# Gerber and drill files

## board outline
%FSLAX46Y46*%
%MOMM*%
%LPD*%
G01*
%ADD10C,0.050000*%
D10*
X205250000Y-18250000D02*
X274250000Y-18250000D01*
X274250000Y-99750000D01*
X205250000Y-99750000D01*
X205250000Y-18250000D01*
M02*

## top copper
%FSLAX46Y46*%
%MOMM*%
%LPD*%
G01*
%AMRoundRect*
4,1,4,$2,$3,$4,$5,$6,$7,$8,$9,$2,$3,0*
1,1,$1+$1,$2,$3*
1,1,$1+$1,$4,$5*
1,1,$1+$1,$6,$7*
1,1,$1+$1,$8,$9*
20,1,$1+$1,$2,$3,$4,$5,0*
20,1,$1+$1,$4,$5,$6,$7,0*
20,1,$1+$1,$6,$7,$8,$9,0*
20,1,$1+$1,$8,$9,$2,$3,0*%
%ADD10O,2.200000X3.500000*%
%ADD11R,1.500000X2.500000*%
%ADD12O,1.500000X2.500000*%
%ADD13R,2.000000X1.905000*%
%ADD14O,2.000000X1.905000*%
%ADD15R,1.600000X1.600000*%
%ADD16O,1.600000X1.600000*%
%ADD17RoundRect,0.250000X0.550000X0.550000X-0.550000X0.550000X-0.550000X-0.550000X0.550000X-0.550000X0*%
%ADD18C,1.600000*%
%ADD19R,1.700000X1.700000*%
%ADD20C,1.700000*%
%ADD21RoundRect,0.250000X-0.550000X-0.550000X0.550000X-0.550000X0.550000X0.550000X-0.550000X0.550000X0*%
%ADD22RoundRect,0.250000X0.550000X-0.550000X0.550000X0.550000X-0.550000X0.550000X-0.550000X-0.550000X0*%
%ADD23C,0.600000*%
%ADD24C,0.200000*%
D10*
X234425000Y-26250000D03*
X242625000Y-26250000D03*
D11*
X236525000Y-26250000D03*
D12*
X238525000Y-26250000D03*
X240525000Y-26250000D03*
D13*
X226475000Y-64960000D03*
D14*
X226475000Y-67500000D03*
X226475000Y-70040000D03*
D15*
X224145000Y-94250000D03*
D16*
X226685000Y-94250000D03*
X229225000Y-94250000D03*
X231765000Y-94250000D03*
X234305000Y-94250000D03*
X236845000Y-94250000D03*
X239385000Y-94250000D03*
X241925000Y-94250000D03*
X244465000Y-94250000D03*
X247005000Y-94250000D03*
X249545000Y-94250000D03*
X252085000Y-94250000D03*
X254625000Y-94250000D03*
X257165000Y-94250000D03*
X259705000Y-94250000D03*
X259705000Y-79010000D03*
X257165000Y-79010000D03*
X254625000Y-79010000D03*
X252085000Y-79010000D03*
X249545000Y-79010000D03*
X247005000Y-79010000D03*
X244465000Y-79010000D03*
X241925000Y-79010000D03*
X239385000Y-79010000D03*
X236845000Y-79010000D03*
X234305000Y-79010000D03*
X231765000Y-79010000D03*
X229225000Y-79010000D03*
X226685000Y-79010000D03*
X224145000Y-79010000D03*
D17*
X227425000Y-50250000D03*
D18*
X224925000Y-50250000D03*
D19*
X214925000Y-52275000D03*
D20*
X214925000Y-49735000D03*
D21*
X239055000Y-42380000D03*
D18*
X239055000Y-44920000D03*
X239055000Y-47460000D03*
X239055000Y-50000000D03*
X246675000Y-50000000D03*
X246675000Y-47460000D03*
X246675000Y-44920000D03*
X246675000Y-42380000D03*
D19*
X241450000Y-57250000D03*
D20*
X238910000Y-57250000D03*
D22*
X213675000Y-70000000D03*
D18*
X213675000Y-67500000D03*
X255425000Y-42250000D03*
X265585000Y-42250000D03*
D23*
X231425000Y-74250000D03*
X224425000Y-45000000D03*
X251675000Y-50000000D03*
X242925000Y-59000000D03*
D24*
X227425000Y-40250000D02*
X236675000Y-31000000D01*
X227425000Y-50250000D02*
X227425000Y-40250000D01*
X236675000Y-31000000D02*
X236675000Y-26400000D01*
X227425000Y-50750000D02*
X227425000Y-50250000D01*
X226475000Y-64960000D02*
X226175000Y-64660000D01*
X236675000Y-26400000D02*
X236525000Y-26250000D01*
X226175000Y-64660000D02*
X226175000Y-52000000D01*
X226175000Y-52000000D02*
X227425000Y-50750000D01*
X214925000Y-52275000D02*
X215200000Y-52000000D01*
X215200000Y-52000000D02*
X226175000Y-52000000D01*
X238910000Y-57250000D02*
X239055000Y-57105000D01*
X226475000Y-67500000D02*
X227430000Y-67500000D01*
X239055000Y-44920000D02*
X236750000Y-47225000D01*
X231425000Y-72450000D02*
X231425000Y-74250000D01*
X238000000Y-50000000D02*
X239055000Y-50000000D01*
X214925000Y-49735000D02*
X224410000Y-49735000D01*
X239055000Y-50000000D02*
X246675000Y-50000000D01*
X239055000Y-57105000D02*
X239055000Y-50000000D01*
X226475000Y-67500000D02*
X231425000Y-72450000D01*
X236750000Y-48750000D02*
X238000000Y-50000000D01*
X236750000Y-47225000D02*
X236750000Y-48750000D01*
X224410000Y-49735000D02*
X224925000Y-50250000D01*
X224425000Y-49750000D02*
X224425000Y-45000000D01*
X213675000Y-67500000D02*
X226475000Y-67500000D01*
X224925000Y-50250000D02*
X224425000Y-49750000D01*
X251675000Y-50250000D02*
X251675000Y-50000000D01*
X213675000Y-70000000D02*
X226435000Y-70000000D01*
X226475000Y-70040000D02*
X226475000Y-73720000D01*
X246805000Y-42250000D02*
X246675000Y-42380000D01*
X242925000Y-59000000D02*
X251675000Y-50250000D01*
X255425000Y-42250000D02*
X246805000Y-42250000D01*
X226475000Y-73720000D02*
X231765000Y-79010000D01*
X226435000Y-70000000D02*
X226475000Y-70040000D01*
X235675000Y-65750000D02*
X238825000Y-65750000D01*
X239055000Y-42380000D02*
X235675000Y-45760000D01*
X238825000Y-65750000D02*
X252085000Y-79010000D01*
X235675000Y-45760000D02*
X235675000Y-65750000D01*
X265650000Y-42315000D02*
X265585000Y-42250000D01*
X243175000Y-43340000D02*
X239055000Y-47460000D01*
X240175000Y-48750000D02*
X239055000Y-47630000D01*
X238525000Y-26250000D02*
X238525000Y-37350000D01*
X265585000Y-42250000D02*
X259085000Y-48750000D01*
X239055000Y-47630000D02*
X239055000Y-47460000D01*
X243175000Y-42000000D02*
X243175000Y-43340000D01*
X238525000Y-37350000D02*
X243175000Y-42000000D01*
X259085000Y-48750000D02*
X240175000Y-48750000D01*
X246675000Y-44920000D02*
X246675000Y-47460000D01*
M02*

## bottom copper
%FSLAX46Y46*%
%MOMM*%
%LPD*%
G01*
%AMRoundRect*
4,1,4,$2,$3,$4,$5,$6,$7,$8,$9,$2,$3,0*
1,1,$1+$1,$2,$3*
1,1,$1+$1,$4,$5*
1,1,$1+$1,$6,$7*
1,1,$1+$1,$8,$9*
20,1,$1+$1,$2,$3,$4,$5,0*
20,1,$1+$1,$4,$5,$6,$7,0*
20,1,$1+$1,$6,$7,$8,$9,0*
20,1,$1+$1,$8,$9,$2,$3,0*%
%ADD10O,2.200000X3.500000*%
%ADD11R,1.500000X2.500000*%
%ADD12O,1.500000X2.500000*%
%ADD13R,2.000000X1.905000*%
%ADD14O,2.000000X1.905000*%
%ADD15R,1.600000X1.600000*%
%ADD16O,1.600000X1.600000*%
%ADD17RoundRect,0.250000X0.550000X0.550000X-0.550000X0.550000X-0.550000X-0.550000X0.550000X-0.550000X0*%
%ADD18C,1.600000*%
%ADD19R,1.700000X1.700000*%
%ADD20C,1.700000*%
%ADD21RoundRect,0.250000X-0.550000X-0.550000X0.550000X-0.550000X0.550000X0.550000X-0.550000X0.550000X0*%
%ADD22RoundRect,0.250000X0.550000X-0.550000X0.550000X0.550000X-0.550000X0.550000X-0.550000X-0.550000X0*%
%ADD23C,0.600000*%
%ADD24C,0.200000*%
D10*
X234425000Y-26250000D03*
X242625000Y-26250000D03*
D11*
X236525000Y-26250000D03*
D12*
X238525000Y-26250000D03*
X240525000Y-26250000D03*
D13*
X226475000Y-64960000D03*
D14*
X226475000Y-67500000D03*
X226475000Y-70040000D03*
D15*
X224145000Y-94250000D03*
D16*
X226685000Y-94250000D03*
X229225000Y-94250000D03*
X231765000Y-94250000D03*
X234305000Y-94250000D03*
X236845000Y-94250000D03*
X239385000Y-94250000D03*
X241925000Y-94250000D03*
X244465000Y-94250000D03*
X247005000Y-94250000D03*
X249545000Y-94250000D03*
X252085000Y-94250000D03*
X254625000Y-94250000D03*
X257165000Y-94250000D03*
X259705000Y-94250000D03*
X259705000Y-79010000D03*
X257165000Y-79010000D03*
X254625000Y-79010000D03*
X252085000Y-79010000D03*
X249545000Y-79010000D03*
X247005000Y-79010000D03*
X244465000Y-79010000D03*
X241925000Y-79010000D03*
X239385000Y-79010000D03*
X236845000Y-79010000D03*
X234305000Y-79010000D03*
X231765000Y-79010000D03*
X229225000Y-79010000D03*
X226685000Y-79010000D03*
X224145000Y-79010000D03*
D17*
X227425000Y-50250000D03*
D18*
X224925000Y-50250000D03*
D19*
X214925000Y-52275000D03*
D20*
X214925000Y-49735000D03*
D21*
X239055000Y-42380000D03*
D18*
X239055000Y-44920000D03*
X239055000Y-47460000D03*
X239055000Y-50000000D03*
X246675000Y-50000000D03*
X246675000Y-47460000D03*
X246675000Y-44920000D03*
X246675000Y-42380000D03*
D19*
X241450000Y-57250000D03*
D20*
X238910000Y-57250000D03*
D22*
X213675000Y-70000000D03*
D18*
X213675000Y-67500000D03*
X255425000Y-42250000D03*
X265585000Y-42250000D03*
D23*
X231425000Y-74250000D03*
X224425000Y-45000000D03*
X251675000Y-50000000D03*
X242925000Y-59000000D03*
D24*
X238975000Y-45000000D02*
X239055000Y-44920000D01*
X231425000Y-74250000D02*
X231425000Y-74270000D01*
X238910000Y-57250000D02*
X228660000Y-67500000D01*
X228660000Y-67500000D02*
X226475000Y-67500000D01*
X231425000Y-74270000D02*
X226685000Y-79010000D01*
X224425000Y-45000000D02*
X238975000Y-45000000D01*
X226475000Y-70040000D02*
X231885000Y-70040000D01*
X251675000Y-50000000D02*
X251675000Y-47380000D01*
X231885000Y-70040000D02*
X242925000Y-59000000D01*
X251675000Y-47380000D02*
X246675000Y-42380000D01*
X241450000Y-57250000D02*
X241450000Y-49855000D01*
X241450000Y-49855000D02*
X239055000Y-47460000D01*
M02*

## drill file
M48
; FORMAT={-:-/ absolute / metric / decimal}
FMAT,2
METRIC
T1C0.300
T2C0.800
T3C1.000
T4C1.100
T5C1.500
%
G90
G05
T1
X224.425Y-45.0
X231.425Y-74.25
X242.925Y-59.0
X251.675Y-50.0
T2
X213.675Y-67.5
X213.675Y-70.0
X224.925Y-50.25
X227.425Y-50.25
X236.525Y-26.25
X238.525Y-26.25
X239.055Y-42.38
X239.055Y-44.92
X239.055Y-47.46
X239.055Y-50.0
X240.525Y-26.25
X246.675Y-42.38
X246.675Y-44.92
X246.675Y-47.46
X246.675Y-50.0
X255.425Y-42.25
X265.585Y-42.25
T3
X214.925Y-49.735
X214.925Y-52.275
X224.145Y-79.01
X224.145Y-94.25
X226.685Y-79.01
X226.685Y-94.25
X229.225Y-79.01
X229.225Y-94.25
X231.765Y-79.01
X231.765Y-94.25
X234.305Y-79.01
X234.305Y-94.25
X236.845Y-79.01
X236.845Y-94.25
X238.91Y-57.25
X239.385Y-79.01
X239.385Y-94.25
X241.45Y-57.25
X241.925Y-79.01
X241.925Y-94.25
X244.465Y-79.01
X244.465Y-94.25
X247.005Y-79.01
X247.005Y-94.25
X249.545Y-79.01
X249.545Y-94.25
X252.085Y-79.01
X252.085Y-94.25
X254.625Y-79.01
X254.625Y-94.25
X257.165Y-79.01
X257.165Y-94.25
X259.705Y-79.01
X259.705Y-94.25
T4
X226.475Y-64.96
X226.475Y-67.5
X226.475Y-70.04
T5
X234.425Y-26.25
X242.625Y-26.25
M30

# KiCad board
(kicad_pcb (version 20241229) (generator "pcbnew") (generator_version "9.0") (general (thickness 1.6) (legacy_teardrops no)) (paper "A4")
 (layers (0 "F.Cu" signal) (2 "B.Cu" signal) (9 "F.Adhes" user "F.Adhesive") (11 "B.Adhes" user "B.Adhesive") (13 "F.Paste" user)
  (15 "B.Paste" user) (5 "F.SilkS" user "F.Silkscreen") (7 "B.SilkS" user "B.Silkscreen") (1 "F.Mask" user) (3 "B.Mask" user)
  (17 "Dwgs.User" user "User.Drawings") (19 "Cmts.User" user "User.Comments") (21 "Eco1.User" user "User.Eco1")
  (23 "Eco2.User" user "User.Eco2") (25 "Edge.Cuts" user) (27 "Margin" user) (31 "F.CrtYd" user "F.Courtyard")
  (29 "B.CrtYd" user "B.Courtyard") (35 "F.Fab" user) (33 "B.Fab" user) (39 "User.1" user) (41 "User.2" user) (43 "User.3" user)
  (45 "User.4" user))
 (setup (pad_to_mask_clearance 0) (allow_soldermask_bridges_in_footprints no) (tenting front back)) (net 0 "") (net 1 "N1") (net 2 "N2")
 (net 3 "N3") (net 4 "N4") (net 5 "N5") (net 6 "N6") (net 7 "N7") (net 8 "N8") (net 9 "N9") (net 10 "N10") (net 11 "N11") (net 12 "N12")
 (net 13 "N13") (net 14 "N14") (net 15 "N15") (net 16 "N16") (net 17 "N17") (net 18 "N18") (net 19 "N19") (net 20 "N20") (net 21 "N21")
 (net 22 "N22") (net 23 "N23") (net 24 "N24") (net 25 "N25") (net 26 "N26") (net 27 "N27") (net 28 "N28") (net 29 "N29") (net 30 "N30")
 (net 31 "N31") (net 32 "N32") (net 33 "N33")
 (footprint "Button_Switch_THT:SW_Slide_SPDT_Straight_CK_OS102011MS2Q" (layer "F.Cu") (at 236.525 26.25)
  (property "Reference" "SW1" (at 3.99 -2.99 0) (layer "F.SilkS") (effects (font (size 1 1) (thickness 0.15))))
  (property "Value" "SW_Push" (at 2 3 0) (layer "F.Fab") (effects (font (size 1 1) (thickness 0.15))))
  (pad "" thru_hole oval (at -2.1 0) (size 2.2 3.5) (drill 1.5) (layers "*.Cu" "*.Mask") (remove_unused_layers no))
  (pad "" thru_hole oval (at 6.1 0) (size 2.2 3.5) (drill 1.5) (layers "*.Cu" "*.Mask") (remove_unused_layers no))
  (pad "1" thru_hole rect (at 0 0) (size 1.5 2.5) (drill 0.8) (layers "*.Cu" "*.Mask") (remove_unused_layers no) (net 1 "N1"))
  (pad "2" thru_hole oval (at 2 0) (size 1.5 2.5) (drill 0.8) (layers "*.Cu" "*.Mask") (remove_unused_layers no) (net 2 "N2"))
  (pad "3" thru_hole oval (at 4 0) (size 1.5 2.5) (drill 0.8) (layers "*.Cu" "*.Mask") (remove_unused_layers no)))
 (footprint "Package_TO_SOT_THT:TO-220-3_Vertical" (layer "F.Cu") (at 226.475 64.96 -90)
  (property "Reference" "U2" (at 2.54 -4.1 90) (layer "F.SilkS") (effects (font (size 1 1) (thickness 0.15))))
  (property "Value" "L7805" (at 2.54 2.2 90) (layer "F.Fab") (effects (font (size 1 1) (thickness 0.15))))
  (pad "1" thru_hole rect (at 0 0 270) (size 1.905 2) (drill 1.1) (layers "*.Cu" "*.Mask") (remove_unused_layers no) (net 1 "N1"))
  (pad "2" thru_hole oval (at 2.54 0 270) (size 1.905 2) (drill 1.1) (layers "*.Cu" "*.Mask") (remove_unused_layers no) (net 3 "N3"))
  (pad "3" thru_hole oval (at 5.08 0 270) (size 1.905 2) (drill 1.1) (layers "*.Cu" "*.Mask") (remove_unused_layers no) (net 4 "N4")))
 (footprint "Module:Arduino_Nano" (layer "F.Cu") (at 224.145 94.25 90)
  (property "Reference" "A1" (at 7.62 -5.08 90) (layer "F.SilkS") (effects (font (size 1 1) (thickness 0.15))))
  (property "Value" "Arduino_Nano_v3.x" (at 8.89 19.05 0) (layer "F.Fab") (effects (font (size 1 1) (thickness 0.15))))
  (pad "1" thru_hole rect (at 0 0 90) (size 1.6 1.6) (drill 1) (layers "*.Cu" "*.Mask") (remove_unused_layers no) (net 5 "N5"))
  (pad "2" thru_hole oval (at 0 2.54 90) (size 1.6 1.6) (drill 1) (layers "*.Cu" "*.Mask") (remove_unused_layers no) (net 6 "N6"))
  (pad "3" thru_hole oval (at 0 5.08 90) (size 1.6 1.6) (drill 1) (layers "*.Cu" "*.Mask") (remove_unused_layers no) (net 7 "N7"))
  (pad "4" thru_hole oval (at 0 7.62 90) (size 1.6 1.6) (drill 1) (layers "*.Cu" "*.Mask") (remove_unused_layers no) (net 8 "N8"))
  (pad "5" thru_hole oval (at 0 10.16 90) (size 1.6 1.6) (drill 1) (layers "*.Cu" "*.Mask") (remove_unused_layers no) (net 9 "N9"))
  (pad "6" thru_hole oval (at 0 12.7 90) (size 1.6 1.6) (drill 1) (layers "*.Cu" "*.Mask") (remove_unused_layers no) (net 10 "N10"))
  (pad "7" thru_hole oval (at 0 15.24 90) (size 1.6 1.6) (drill 1) (layers "*.Cu" "*.Mask") (remove_unused_layers no) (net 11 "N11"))
  (pad "8" thru_hole oval (at 0 17.78 90) (size 1.6 1.6) (drill 1) (layers "*.Cu" "*.Mask") (remove_unused_layers no) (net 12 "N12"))
  (pad "9" thru_hole oval (at 0 20.32 90) (size 1.6 1.6) (drill 1) (layers "*.Cu" "*.Mask") (remove_unused_layers no) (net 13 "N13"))
  (pad "10" thru_hole oval (at 0 22.86 90) (size 1.6 1.6) (drill 1) (layers "*.Cu" "*.Mask") (remove_unused_layers no) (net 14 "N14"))
  (pad "11" thru_hole oval (at 0 25.4 90) (size 1.6 1.6) (drill 1) (layers "*.Cu" "*.Mask") (remove_unused_layers no) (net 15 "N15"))
  (pad "12" thru_hole oval (at 0 27.94 90) (size 1.6 1.6) (drill 1) (layers "*.Cu" "*.Mask") (remove_unused_layers no) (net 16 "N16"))
  (pad "13" thru_hole oval (at 0 30.48 90) (size 1.6 1.6) (drill 1) (layers "*.Cu" "*.Mask") (remove_unused_layers no) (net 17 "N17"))
  (pad "14" thru_hole oval (at 0 33.02 90) (size 1.6 1.6) (drill 1) (layers "*.Cu" "*.Mask") (remove_unused_layers no) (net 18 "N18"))
  (pad "15" thru_hole oval (at 0 35.56 90) (size 1.6 1.6) (drill 1) (layers "*.Cu" "*.Mask") (remove_unused_layers no) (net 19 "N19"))
  (pad "16" thru_hole oval (at 15.24 35.56 90) (size 1.6 1.6) (drill 1) (layers "*.Cu" "*.Mask") (remove_unused_layers no) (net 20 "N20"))
  (pad "17" thru_hole oval (at 15.24 33.02 90) (size 1.6 1.6) (drill 1) (layers "*.Cu" "*.Mask") (remove_unused_layers no) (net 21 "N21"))
  (pad "18" thru_hole oval (at 15.24 30.48 90) (size 1.6 1.6) (drill 1) (layers "*.Cu" "*.Mask") (remove_unused_layers no) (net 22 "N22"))
  (pad "19" thru_hole oval (at 15.24 27.94 90) (size 1.6 1.6) (drill 1) (layers "*.Cu" "*.Mask") (remove_unused_layers no) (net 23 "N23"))
  (pad "20" thru_hole oval (at 15.24 25.4 90) (size 1.6 1.6) (drill 1) (layers "*.Cu" "*.Mask") (remove_unused_layers no) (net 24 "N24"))
  (pad "21" thru_hole oval (at 15.24 22.86 90) (size 1.6 1.6) (drill 1) (layers "*.Cu" "*.Mask") (remove_unused_layers no) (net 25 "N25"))
  (pad "22" thru_hole oval (at 15.24 20.32 90) (size 1.6 1.6) (drill 1) (layers "*.Cu" "*.Mask") (remove_unused_layers no) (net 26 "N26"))
  (pad "23" thru_hole oval (at 15.24 17.78 90) (size 1.6 1.6) (drill 1) (layers "*.Cu" "*.Mask") (remove_unused_layers no) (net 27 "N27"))
  (pad "24" thru_hole oval (at 15.24 15.24 90) (size 1.6 1.6) (drill 1) (layers "*.Cu" "*.Mask") (remove_unused_layers no) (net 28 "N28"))
  (pad "25" thru_hole oval (at 15.24 12.7 90) (size 1.6 1.6) (drill 1) (layers "*.Cu" "*.Mask") (remove_unused_layers no) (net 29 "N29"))
  (pad "26" thru_hole oval (at 15.24 10.16 90) (size 1.6 1.6) (drill 1) (layers "*.Cu" "*.Mask") (remove_unused_layers no) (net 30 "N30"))
  (pad "27" thru_hole oval (at 15.24 7.62 90) (size 1.6 1.6) (drill 1) (layers "*.Cu" "*.Mask") (remove_unused_layers no) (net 4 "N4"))
  (pad "28" thru_hole oval (at 15.24 5.08 90) (size 1.6 1.6) (drill 1) (layers "*.Cu" "*.Mask") (remove_unused_layers no) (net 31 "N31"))
  (pad "29" thru_hole oval (at 15.24 2.54 90) (size 1.6 1.6) (drill 1) (layers "*.Cu" "*.Mask") (remove_unused_layers no) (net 3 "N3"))
  (pad "30" thru_hole oval (at 15.24 0 90) (size 1.6 1.6) (drill 1) (layers "*.Cu" "*.Mask") (remove_unused_layers no) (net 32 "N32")))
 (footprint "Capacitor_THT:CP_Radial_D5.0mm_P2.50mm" (layer "F.Cu") (at 227.425 50.25 180)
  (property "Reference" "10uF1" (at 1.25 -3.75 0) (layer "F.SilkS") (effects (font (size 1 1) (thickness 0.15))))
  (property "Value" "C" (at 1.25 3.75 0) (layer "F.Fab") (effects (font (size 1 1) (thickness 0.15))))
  (pad "1" thru_hole roundrect (at 0 0 180) (size 1.6 1.6) (drill 0.8) (layers "*.Cu" "*.Mask") (remove_unused_layers no)
   (roundrect_rratio 0.15625) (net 1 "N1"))
  (pad "2" thru_hole circle (at 2.5 0 180) (size 1.6 1.6) (drill 0.8) (layers "*.Cu" "*.Mask") (remove_unused_layers no) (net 3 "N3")))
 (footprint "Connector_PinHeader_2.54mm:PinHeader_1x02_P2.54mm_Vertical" (layer "F.Cu") (at 214.925 52.275 180)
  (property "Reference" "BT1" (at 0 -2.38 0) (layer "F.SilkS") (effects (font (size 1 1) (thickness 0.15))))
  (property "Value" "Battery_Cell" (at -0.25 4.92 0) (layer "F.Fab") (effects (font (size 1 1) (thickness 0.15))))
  (pad "1" thru_hole rect (at 0 0 180) (size 1.7 1.7) (drill 1) (layers "*.Cu" "*.Mask") (remove_unused_layers no) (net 1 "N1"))
  (pad "2" thru_hole circle (at 0 2.54 180) (size 1.7 1.7) (drill 1) (layers "*.Cu" "*.Mask") (remove_unused_layers no) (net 3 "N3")))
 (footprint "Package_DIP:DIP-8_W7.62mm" (layer "F.Cu") (at 239.055 42.38)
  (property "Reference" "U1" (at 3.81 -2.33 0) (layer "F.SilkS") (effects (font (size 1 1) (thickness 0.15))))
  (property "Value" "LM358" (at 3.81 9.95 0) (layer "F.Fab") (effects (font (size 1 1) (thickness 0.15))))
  (pad "1" thru_hole roundrect (at 0 0) (size 1.6 1.6) (drill 0.8) (layers "*.Cu" "*.Mask") (remove_unused_layers no)
   (roundrect_rratio 0.15625) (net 23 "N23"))
  (pad "2" thru_hole circle (at 0 2.54) (size 1.6 1.6) (drill 0.8) (layers "*.Cu" "*.Mask") (remove_unused_layers no) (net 3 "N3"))
  (pad "3" thru_hole circle (at 0 5.08) (size 1.6 1.6) (drill 0.8) (layers "*.Cu" "*.Mask") (remove_unused_layers no) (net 2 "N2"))
  (pad "4" thru_hole circle (at 0 7.62) (size 1.6 1.6) (drill 0.8) (layers "*.Cu" "*.Mask") (remove_unused_layers no) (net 3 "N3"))
  (pad "5" thru_hole circle (at 7.62 7.62) (size 1.6 1.6) (drill 0.8) (layers "*.Cu" "*.Mask") (remove_unused_layers no) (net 3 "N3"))
  (pad "6" thru_hole circle (at 7.62 5.08) (size 1.6 1.6) (drill 0.8) (layers "*.Cu" "*.Mask") (remove_unused_layers no) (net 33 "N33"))
  (pad "7" thru_hole circle (at 7.62 2.54) (size 1.6 1.6) (drill 0.8) (layers "*.Cu" "*.Mask") (remove_unused_layers no) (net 33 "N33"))
  (pad "8" thru_hole circle (at 7.62 0) (size 1.6 1.6) (drill 0.8) (layers "*.Cu" "*.Mask") (remove_unused_layers no) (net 4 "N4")))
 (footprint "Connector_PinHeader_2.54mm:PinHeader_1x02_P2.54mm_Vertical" (layer "F.Cu") (at 241.45 57.25 -90)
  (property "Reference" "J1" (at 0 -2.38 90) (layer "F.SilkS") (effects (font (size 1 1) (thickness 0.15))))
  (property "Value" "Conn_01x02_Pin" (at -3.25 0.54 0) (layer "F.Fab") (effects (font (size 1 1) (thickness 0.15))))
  (pad "1" thru_hole rect (at 0 0 270) (size 1.7 1.7) (drill 1) (layers "*.Cu" "*.Mask") (remove_unused_layers no) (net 2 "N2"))
  (pad "2" thru_hole circle (at 0 2.54 270) (size 1.7 1.7) (drill 1) (layers "*.Cu" "*.Mask") (remove_unused_layers no) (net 3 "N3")))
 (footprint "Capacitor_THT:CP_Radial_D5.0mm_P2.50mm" (layer "F.Cu") (at 213.675 70 90)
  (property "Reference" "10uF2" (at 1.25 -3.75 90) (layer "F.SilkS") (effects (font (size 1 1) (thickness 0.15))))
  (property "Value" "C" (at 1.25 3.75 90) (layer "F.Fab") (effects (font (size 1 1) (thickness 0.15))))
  (pad "1" thru_hole roundrect (at 0 0 90) (size 1.6 1.6) (drill 0.8) (layers "*.Cu" "*.Mask") (remove_unused_layers no)
   (roundrect_rratio 0.15625) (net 4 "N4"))
  (pad "2" thru_hole circle (at 2.5 0 90) (size 1.6 1.6) (drill 0.8) (layers "*.Cu" "*.Mask") (remove_unused_layers no) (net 3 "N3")))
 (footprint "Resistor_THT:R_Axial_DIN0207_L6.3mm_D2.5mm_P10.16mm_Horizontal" (layer "F.Cu") (at 255.425 42.25)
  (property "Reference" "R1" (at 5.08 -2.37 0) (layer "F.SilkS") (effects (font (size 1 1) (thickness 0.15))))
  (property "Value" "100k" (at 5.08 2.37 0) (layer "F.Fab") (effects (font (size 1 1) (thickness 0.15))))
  (pad "1" thru_hole circle (at 0 0) (size 1.6 1.6) (drill 0.8) (layers "*.Cu" "*.Mask") (remove_unused_layers no) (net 4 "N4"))
  (pad "2" thru_hole circle (at 10.16 0) (size 1.6 1.6) (drill 0.8) (layers "*.Cu" "*.Mask") (remove_unused_layers no) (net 2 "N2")))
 (gr_rect (start 205.25 18.25) (end 274.25 99.75) (stroke (width 0.05) (type default)) (fill no) (layer "Edge.Cuts"))
 (segment (start 227.425 40.25) (end 236.675 31) (width 0.2) (layer "F.Cu") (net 1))
 (segment (start 227.425 50.25) (end 227.425 40.25) (width 0.2) (layer "F.Cu") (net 1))
 (segment (start 236.675 31) (end 236.675 26.4) (width 0.2) (layer "F.Cu") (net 1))
 (segment (start 227.425 50.75) (end 227.425 50.25) (width 0.2) (layer "F.Cu") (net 1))
 (segment (start 226.475 64.96) (end 226.175 64.66) (width 0.2) (layer "F.Cu") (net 1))
 (segment (start 236.675 26.4) (end 236.525 26.25) (width 0.2) (layer "F.Cu") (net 1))
 (segment (start 226.175 64.66) (end 226.175 52) (width 0.2) (layer "F.Cu") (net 1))
 (segment (start 226.175 52) (end 227.425 50.75) (width 0.2) (layer "F.Cu") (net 1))
 (segment (start 214.925 52.275) (end 215.2 52) (width 0.2) (layer "F.Cu") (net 1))
 (segment (start 215.2 52) (end 226.175 52) (width 0.2) (layer "F.Cu") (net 1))
 (segment (start 238.91 57.25) (end 239.055 57.105) (width 0.2) (layer "F.Cu") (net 3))
 (segment (start 226.475 67.5) (end 227.43 67.5) (width 0.2) (layer "F.Cu") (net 3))
 (segment (start 239.055 44.92) (end 236.75 47.225) (width 0.2) (layer "F.Cu") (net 3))
 (segment (start 231.425 72.45) (end 231.425 74.25) (width 0.2) (layer "F.Cu") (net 3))
 (segment (start 238 50) (end 239.055 50) (width 0.2) (layer "F.Cu") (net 3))
 (segment (start 214.925 49.735) (end 224.41 49.735) (width 0.2) (layer "F.Cu") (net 3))
 (segment (start 239.055 50) (end 246.675 50) (width 0.2) (layer "F.Cu") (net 3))
 (segment (start 239.055 57.105) (end 239.055 50) (width 0.2) (layer "F.Cu") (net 3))
 (segment (start 226.475 67.5) (end 231.425 72.45) (width 0.2) (layer "F.Cu") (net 3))
 (segment (start 236.75 48.75) (end 238 50) (width 0.2) (layer "F.Cu") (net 3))
 (segment (start 236.75 47.225) (end 236.75 48.75) (width 0.2) (layer "F.Cu") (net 3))
 (segment (start 224.41 49.735) (end 224.925 50.25) (width 0.2) (layer "F.Cu") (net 3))
 (segment (start 224.425 49.75) (end 224.425 45) (width 0.2) (layer "F.Cu") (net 3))
 (segment (start 213.675 67.5) (end 226.475 67.5) (width 0.2) (layer "F.Cu") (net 3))
 (segment (start 224.925 50.25) (end 224.425 49.75) (width 0.2) (layer "F.Cu") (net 3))
 (via (at 231.425 74.25) (size 0.6) (drill 0.3) (layers "F.Cu" "B.Cu") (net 3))
 (via (at 224.425 45) (size 0.6) (drill 0.3) (layers "F.Cu" "B.Cu") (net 3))
 (segment (start 238.975 45) (end 239.055 44.92) (width 0.2) (layer "B.Cu") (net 3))
 (segment (start 231.425 74.25) (end 231.425 74.27) (width 0.2) (layer "B.Cu") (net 3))
 (segment (start 238.91 57.25) (end 228.66 67.5) (width 0.2) (layer "B.Cu") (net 3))
 (segment (start 228.66 67.5) (end 226.475 67.5) (width 0.2) (layer "B.Cu") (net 3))
 (segment (start 231.425 74.27) (end 226.685 79.01) (width 0.2) (layer "B.Cu") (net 3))
 (segment (start 224.425 45) (end 238.975 45) (width 0.2) (layer "B.Cu") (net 3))
 (segment (start 251.675 50.25) (end 251.675 50) (width 0.2) (layer "F.Cu") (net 4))
 (segment (start 213.675 70) (end 226.435 70) (width 0.2) (layer "F.Cu") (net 4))
 (segment (start 226.475 70.04) (end 226.475 73.72) (width 0.2) (layer "F.Cu") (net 4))
 (segment (start 246.805 42.25) (end 246.675 42.38) (width 0.2) (layer "F.Cu") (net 4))
 (segment (start 242.925 59) (end 251.675 50.25) (width 0.2) (layer "F.Cu") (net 4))
 (segment (start 255.425 42.25) (end 246.805 42.25) (width 0.2) (layer "F.Cu") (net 4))
 (segment (start 226.475 73.72) (end 231.765 79.01) (width 0.2) (layer "F.Cu") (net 4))
 (segment (start 226.435 70) (end 226.475 70.04) (width 0.2) (layer "F.Cu") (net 4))
 (via (at 251.675 50) (size 0.6) (drill 0.3) (layers "F.Cu" "B.Cu") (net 4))
 (via (at 242.925 59) (size 0.6) (drill 0.3) (layers "F.Cu" "B.Cu") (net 4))
 (segment (start 226.475 70.04) (end 231.885 70.04) (width 0.2) (layer "B.Cu") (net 4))
 (segment (start 251.675 50) (end 251.675 47.38) (width 0.2) (layer "B.Cu") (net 4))
 (segment (start 231.885 70.04) (end 242.925 59) (width 0.2) (layer "B.Cu") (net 4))
 (segment (start 251.675 47.38) (end 246.675 42.38) (width 0.2) (layer "B.Cu") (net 4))
 (segment (start 235.675 65.75) (end 238.825 65.75) (width 0.2) (layer "F.Cu") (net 23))
 (segment (start 239.055 42.38) (end 235.675 45.76) (width 0.2) (layer "F.Cu") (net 23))
 (segment (start 238.825 65.75) (end 252.085 79.01) (width 0.2) (layer "F.Cu") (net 23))
 (segment (start 235.675 45.76) (end 235.675 65.75) (width 0.2) (layer "F.Cu") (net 23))
 (segment (start 265.65 42.315) (end 265.585 42.25) (width 0.2) (layer "F.Cu") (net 2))
 (segment (start 243.175 43.34) (end 239.055 47.46) (width 0.2) (layer "F.Cu") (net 2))
 (segment (start 240.175 48.75) (end 239.055 47.63) (width 0.2) (layer "F.Cu") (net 2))
 (segment (start 238.525 26.25) (end 238.525 37.35) (width 0.2) (layer "F.Cu") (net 2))
 (segment (start 265.585 42.25) (end 259.085 48.75) (width 0.2) (layer "F.Cu") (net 2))
 (segment (start 239.055 47.63) (end 239.055 47.46) (width 0.2) (layer "F.Cu") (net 2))
 (segment (start 243.175 42) (end 243.175 43.34) (width 0.2) (layer "F.Cu") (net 2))
 (segment (start 238.525 37.35) (end 243.175 42) (width 0.2) (layer "F.Cu") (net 2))
 (segment (start 259.085 48.75) (end 240.175 48.75) (width 0.2) (layer "F.Cu") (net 2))
 (segment (start 241.45 57.25) (end 241.45 49.855) (width 0.2) (layer "B.Cu") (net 2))
 (segment (start 241.45 49.855) (end 239.055 47.46) (width 0.2) (layer "B.Cu") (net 2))
 (segment (start 246.675 44.92) (end 246.675 47.46) (width 0.2) (layer "F.Cu") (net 33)))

